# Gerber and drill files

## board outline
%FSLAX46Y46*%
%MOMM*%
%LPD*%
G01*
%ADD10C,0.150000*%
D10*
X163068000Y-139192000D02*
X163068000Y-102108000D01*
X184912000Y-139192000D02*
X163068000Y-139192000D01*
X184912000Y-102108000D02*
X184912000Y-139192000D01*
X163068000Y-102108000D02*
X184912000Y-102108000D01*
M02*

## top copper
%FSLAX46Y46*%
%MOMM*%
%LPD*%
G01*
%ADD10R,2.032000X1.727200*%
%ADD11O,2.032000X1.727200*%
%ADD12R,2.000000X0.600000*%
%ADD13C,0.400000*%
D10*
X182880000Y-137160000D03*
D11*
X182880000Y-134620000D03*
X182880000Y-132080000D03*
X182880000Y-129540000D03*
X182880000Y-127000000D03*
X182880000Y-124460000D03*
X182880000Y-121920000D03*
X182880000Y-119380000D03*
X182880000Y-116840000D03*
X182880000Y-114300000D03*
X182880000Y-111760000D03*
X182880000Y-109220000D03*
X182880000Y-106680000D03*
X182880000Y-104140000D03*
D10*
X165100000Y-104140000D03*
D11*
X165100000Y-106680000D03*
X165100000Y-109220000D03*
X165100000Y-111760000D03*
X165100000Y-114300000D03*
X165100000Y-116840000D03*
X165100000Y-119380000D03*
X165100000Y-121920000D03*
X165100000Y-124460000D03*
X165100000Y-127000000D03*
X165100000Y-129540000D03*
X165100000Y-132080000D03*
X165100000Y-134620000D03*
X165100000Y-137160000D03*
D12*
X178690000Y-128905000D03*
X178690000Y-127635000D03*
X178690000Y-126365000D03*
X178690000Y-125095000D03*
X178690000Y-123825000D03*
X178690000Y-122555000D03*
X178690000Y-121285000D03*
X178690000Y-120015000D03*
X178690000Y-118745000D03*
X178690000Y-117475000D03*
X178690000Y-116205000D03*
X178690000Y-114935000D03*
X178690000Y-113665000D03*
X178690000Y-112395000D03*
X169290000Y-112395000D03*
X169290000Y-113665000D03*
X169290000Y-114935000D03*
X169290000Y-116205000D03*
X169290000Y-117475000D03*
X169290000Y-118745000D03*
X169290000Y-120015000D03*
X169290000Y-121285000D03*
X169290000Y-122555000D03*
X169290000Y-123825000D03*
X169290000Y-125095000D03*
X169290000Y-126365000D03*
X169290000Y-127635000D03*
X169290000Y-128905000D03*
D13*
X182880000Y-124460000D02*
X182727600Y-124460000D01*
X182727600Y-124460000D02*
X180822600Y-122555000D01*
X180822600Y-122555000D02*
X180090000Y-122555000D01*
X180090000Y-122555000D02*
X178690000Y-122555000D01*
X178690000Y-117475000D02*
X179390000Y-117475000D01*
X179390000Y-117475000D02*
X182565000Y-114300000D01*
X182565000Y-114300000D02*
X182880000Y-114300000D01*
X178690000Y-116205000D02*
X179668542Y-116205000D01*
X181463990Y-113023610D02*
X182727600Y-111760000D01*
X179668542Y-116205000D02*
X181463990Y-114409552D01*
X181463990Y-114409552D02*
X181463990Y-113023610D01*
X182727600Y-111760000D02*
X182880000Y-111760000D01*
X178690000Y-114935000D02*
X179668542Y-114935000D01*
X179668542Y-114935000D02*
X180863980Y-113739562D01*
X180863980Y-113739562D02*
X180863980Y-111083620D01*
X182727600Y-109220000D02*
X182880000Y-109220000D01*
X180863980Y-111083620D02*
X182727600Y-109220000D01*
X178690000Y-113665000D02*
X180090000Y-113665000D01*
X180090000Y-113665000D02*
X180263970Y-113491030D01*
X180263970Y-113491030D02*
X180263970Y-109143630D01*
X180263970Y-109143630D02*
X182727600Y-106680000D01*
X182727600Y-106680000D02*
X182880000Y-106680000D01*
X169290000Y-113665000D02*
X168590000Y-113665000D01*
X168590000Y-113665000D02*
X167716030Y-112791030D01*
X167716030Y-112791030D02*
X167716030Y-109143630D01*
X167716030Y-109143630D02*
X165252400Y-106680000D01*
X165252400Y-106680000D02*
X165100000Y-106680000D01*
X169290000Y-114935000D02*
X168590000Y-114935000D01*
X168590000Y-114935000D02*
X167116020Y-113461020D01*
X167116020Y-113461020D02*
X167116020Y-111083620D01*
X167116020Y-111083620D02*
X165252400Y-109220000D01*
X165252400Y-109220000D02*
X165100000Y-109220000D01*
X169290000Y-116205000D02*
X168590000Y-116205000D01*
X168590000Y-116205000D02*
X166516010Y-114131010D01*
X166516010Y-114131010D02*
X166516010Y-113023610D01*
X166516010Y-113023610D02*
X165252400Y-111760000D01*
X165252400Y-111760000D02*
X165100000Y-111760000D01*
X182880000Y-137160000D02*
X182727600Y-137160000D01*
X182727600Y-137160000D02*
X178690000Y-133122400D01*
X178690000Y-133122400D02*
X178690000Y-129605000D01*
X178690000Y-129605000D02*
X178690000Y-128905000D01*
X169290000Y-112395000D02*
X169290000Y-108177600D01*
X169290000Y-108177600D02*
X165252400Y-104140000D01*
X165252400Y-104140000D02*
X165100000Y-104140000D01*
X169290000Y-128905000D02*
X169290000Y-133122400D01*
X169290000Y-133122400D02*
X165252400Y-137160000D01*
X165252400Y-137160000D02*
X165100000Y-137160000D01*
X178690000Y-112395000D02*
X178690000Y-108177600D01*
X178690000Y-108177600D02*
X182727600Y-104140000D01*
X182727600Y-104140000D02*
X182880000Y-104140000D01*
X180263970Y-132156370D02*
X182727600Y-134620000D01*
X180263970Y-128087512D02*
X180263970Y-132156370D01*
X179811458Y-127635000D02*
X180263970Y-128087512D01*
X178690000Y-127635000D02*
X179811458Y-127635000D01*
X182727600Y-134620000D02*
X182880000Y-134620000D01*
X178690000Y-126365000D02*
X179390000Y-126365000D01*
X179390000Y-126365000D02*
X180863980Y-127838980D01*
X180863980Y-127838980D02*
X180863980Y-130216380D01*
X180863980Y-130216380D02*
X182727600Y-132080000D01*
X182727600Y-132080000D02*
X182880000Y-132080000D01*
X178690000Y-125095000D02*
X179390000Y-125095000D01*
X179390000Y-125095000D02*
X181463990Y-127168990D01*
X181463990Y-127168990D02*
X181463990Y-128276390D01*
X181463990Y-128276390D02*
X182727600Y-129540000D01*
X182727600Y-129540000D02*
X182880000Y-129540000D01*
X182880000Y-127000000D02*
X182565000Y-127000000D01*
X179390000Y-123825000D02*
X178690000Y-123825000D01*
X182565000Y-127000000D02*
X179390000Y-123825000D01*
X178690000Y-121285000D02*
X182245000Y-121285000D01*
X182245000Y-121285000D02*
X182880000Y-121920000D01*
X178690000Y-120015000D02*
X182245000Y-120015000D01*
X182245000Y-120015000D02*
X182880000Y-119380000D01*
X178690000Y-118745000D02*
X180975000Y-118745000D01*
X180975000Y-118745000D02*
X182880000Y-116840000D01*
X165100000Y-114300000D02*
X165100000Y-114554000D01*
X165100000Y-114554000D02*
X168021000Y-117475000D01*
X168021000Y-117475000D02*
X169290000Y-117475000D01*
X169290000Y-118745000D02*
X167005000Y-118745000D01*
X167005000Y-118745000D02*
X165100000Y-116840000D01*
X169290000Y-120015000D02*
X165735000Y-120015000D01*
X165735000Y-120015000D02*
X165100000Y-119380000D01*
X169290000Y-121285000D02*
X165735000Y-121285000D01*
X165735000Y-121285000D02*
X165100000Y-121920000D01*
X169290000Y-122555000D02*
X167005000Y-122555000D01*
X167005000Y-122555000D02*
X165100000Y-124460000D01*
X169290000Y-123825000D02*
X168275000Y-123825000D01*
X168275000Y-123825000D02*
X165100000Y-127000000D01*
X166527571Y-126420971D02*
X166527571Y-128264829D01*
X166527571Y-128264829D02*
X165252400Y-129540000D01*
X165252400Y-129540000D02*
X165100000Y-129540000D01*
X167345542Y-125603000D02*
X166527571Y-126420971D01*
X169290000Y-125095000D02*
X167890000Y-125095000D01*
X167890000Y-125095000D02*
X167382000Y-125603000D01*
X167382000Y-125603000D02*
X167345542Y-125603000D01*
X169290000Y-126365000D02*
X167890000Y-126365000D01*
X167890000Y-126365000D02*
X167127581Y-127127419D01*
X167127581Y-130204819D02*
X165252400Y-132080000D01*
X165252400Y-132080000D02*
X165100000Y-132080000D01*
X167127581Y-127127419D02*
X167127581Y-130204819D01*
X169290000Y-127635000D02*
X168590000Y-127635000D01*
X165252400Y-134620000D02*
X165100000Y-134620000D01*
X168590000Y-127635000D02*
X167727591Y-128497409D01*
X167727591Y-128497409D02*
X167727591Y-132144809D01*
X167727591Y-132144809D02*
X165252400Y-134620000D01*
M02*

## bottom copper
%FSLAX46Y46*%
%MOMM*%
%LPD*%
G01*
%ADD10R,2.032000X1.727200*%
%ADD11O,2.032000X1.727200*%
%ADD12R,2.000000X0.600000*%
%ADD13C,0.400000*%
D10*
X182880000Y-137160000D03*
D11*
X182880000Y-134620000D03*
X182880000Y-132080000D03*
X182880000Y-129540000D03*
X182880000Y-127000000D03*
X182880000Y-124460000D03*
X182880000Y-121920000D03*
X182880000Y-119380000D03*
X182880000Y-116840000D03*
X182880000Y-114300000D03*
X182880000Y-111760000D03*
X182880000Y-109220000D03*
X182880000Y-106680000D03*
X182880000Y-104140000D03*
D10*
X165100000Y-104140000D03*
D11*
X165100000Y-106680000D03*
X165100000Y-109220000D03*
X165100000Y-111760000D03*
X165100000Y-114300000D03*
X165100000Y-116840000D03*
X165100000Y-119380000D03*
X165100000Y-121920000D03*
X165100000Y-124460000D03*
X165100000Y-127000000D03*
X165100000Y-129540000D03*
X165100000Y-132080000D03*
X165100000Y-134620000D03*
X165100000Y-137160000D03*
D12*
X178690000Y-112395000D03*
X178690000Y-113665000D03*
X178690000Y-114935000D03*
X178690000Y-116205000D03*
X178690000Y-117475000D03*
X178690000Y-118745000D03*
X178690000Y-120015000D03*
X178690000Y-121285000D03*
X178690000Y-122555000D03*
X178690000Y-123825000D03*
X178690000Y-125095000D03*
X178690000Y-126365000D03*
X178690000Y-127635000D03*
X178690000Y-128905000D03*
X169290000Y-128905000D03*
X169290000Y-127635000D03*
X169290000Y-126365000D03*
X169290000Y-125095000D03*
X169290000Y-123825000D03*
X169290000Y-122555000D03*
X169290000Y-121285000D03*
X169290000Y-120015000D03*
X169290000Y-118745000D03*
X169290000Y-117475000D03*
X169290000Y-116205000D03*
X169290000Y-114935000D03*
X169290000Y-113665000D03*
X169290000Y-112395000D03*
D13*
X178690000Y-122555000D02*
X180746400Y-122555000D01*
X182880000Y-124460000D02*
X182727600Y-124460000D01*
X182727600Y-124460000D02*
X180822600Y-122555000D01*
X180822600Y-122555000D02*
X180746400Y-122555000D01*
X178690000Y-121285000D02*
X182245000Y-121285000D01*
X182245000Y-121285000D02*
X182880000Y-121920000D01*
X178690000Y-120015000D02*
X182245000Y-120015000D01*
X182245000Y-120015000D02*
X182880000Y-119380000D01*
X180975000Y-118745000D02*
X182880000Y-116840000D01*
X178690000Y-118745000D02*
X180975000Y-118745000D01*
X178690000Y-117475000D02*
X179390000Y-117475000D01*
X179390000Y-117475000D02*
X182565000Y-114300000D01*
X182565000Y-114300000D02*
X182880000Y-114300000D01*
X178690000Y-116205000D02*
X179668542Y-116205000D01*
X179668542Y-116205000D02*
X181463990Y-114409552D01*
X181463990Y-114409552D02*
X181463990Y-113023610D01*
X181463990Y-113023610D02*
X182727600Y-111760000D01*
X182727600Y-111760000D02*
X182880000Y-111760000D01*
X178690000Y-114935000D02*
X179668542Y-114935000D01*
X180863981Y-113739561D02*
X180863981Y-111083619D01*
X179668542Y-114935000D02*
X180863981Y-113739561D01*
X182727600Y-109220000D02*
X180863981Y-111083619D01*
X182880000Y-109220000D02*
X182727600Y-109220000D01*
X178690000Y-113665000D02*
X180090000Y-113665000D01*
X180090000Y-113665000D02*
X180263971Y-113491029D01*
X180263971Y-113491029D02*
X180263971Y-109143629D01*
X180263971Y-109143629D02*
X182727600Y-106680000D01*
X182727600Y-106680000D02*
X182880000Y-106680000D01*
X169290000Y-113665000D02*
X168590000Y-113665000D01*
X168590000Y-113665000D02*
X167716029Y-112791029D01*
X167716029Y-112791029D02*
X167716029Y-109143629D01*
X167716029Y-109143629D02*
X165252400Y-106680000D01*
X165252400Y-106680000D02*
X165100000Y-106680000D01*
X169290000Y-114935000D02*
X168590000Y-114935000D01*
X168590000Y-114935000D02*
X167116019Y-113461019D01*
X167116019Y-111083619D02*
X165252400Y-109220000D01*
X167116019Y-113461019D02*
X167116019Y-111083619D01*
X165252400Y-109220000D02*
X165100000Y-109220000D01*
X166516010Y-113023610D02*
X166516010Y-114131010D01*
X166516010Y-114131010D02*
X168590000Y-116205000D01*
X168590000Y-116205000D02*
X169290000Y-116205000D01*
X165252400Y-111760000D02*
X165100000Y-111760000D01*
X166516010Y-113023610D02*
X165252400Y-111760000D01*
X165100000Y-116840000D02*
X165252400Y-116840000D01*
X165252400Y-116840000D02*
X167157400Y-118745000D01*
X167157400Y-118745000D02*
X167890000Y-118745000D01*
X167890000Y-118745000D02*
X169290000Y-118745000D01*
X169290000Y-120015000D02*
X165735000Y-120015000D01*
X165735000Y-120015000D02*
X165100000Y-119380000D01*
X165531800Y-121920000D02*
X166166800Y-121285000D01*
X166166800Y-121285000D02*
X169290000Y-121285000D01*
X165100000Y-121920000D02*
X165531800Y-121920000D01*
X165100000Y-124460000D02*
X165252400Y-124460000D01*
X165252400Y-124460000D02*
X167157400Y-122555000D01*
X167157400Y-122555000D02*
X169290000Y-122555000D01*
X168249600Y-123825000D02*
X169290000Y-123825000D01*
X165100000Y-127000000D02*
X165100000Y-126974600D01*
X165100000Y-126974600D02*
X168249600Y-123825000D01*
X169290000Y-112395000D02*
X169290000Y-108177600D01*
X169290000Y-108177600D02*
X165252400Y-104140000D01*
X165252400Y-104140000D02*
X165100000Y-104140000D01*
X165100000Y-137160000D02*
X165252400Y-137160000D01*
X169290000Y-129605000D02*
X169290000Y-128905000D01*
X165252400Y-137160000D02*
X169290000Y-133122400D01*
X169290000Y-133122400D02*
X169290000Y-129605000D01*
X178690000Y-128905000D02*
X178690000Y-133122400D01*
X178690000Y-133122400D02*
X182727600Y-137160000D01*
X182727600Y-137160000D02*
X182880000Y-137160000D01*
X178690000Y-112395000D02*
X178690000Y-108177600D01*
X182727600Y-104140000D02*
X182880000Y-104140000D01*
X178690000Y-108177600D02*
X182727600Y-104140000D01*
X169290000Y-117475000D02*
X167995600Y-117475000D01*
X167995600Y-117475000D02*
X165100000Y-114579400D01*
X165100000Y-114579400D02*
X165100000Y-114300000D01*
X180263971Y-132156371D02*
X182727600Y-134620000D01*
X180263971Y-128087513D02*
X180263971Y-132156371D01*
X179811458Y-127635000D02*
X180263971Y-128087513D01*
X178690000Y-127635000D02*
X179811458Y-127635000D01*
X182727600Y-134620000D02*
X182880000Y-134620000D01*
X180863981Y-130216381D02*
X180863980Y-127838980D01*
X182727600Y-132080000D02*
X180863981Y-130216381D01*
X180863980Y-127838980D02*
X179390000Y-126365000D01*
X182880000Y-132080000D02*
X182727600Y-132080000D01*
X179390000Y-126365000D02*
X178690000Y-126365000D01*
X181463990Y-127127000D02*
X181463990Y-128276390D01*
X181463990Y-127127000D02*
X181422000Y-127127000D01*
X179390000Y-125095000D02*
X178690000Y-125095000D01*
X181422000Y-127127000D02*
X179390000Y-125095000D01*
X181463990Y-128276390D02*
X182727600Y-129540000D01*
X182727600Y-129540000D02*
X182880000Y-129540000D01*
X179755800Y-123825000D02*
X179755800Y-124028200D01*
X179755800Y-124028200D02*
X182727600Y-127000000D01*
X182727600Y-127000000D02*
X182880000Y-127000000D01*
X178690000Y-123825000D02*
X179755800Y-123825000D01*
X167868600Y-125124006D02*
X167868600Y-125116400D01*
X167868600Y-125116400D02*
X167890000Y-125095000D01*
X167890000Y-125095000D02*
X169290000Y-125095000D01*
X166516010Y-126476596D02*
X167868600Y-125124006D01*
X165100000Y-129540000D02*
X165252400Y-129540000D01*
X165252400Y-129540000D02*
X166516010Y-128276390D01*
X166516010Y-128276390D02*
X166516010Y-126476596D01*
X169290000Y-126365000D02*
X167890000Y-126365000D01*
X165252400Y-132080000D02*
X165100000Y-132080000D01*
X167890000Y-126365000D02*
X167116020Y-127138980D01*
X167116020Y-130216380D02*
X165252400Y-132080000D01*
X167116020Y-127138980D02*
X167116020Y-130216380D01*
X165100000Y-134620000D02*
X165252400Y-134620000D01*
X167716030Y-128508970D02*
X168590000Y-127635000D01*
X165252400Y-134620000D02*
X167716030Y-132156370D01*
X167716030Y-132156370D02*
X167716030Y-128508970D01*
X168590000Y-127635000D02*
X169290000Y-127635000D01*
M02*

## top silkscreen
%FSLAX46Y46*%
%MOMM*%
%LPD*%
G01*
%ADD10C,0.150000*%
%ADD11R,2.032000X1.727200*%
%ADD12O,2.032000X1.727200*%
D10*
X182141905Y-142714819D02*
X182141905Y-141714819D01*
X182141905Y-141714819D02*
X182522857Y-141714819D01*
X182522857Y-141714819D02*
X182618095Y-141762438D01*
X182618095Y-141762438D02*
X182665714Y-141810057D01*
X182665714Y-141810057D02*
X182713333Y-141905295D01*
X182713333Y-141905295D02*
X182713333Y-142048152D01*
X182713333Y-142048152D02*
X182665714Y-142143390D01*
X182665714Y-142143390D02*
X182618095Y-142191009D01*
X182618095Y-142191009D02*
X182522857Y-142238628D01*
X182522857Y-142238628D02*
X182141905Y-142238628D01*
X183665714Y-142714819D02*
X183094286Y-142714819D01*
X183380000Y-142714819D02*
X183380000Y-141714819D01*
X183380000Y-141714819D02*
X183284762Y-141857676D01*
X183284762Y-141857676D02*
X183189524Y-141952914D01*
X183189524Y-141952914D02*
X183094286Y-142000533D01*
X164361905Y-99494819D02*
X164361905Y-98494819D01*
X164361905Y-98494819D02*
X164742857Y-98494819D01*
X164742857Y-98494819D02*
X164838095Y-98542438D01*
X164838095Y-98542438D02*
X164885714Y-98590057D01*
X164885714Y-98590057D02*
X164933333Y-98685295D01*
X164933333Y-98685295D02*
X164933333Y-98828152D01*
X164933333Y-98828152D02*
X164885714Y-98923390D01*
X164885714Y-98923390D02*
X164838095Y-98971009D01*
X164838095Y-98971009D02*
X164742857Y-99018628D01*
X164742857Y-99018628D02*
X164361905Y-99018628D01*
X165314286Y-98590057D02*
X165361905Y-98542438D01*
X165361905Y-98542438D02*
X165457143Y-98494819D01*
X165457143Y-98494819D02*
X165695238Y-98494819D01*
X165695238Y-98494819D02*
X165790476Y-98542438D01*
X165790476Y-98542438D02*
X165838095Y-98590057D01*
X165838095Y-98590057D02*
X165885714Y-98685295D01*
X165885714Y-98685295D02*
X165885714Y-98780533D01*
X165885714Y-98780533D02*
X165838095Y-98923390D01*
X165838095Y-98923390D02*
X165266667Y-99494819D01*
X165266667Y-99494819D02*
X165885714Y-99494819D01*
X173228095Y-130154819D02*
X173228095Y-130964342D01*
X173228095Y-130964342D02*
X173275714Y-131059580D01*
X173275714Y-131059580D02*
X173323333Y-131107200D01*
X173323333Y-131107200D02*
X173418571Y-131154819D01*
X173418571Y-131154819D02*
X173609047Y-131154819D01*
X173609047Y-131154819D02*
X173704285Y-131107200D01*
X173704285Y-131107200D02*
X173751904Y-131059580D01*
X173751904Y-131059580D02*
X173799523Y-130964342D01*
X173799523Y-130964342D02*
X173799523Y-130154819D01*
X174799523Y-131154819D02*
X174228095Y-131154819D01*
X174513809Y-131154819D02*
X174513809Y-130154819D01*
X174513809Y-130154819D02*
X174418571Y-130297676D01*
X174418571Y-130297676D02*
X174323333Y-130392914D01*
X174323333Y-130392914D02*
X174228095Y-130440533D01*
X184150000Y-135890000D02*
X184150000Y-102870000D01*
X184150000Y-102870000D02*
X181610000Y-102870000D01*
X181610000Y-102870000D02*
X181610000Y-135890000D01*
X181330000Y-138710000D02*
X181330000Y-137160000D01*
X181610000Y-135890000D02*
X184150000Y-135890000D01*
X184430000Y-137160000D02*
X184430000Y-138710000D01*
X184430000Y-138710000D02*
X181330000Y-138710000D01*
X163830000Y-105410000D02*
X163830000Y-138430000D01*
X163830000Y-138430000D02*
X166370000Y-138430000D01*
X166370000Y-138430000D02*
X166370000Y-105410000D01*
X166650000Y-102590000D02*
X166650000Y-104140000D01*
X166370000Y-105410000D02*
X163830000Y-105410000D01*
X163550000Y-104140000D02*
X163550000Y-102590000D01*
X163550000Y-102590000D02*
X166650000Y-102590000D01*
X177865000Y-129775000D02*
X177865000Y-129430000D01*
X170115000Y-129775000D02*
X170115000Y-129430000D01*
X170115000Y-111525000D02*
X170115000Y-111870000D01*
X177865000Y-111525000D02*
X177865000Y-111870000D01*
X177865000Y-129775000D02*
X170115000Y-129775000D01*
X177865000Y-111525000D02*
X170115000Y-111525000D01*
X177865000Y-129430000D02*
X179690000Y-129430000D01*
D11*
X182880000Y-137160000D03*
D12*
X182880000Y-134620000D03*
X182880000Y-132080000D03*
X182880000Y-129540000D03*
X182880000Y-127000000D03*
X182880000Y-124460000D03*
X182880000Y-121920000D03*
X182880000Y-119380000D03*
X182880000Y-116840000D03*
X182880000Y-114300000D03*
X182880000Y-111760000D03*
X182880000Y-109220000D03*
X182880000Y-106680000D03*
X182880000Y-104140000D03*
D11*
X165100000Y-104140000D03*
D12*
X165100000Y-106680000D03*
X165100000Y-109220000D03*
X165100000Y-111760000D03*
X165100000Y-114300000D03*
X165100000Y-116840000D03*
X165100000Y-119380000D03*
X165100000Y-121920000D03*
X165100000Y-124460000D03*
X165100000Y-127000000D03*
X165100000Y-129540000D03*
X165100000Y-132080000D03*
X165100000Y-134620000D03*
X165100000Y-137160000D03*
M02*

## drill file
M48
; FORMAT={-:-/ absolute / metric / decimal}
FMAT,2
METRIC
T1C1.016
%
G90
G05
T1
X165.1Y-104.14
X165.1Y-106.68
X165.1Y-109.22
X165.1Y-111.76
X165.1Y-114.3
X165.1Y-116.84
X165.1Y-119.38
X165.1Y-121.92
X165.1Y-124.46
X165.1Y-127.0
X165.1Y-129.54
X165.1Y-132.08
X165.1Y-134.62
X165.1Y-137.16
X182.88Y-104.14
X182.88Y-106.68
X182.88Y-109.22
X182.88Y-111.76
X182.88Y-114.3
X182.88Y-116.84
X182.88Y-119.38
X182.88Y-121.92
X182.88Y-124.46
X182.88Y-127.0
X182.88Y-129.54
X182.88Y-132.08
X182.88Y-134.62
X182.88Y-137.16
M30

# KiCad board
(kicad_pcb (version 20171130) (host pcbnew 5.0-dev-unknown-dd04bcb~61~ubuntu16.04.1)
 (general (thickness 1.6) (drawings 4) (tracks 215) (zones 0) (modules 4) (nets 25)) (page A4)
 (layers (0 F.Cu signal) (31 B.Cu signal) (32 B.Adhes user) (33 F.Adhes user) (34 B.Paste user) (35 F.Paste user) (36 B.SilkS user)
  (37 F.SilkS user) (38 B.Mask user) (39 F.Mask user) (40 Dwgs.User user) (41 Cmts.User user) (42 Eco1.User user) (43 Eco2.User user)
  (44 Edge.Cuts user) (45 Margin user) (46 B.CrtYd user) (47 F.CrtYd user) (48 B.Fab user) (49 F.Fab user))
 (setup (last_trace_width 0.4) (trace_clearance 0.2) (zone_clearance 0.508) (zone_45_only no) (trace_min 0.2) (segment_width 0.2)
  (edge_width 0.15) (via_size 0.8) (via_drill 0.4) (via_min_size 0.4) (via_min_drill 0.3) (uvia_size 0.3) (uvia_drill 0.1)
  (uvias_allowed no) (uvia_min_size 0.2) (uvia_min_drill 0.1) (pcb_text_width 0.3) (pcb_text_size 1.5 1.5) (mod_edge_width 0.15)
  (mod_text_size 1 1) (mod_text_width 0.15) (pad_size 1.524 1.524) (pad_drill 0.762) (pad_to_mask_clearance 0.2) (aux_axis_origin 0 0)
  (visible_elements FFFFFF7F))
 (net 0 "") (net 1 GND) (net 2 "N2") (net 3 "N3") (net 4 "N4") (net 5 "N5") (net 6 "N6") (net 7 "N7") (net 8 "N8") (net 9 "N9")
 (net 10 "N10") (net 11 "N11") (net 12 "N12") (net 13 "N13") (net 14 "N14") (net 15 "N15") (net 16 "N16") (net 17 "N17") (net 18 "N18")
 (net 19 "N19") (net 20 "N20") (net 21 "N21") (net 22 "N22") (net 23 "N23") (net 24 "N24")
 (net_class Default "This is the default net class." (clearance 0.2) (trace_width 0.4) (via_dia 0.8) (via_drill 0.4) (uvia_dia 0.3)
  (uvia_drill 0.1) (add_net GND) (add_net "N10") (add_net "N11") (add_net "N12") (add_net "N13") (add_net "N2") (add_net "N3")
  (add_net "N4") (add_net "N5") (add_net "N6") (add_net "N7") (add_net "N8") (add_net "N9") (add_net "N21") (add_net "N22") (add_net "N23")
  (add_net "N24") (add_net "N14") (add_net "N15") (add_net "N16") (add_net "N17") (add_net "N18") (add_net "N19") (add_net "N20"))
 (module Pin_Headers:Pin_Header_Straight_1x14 (layer F.Cu) (at 182.88 137.16 180)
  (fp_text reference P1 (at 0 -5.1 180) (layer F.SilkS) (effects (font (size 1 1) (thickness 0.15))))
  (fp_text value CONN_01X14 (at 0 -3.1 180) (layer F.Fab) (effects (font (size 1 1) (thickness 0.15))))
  (fp_line (start -1.27 1.27) (end -1.27 34.29) (layer F.SilkS) (width 0.15))
  (fp_line (start -1.27 34.29) (end 1.27 34.29) (layer F.SilkS) (width 0.15))
  (fp_line (start 1.27 34.29) (end 1.27 1.27) (layer F.SilkS) (width 0.15))
  (fp_line (start 1.55 -1.55) (end 1.55 0) (layer F.SilkS) (width 0.15))
  (fp_line (start 1.27 1.27) (end -1.27 1.27) (layer F.SilkS) (width 0.15))
  (fp_line (start -1.55 0) (end -1.55 -1.55) (layer F.SilkS) (width 0.15))
  (fp_line (start -1.55 -1.55) (end 1.55 -1.55) (layer F.SilkS) (width 0.15))
  (pad 1 thru_hole rect (at 0 0 180) (size 2.032 1.7272) (drill 1.016) (layers *.Cu *.Mask F.SilkS) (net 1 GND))
  (pad 2 thru_hole oval (at 0 2.54 180) (size 2.032 1.7272) (drill 1.016) (layers *.Cu *.Mask F.SilkS) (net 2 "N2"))
  (pad 3 thru_hole oval (at 0 5.08 180) (size 2.032 1.7272) (drill 1.016) (layers *.Cu *.Mask F.SilkS) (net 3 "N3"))
  (pad 4 thru_hole oval (at 0 7.62 180) (size 2.032 1.7272) (drill 1.016) (layers *.Cu *.Mask F.SilkS) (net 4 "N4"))
  (pad 5 thru_hole oval (at 0 10.16 180) (size 2.032 1.7272) (drill 1.016) (layers *.Cu *.Mask F.SilkS) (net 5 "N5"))
  (pad 6 thru_hole oval (at 0 12.7 180) (size 2.032 1.7272) (drill 1.016) (layers *.Cu *.Mask F.SilkS) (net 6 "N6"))
  (pad 7 thru_hole oval (at 0 15.24 180) (size 2.032 1.7272) (drill 1.016) (layers *.Cu *.Mask F.SilkS) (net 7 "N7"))
  (pad 8 thru_hole oval (at 0 17.78 180) (size 2.032 1.7272) (drill 1.016) (layers *.Cu *.Mask F.SilkS) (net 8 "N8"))
  (pad 9 thru_hole oval (at 0 20.32 180) (size 2.032 1.7272) (drill 1.016) (layers *.Cu *.Mask F.SilkS) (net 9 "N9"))
  (pad 10 thru_hole oval (at 0 22.86 180) (size 2.032 1.7272) (drill 1.016) (layers *.Cu *.Mask F.SilkS) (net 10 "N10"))
  (pad 11 thru_hole oval (at 0 25.4 180) (size 2.032 1.7272) (drill 1.016) (layers *.Cu *.Mask F.SilkS) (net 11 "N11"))
  (pad 12 thru_hole oval (at 0 27.94 180) (size 2.032 1.7272) (drill 1.016) (layers *.Cu *.Mask F.SilkS) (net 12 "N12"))
  (pad 13 thru_hole oval (at 0 30.48 180) (size 2.032 1.7272) (drill 1.016) (layers *.Cu *.Mask F.SilkS) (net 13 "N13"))
  (pad 14 thru_hole oval (at 0 33.02 180) (size 2.032 1.7272) (drill 1.016) (layers *.Cu *.Mask F.SilkS) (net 1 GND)))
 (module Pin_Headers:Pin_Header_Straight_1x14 (layer F.Cu) (at 165.1 104.14)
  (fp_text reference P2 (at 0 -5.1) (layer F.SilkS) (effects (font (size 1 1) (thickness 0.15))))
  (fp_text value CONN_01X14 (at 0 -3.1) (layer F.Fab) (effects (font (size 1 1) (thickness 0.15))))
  (fp_line (start -1.27 1.27) (end -1.27 34.29) (layer F.SilkS) (width 0.15))
  (fp_line (start -1.27 34.29) (end 1.27 34.29) (layer F.SilkS) (width 0.15))
  (fp_line (start 1.27 34.29) (end 1.27 1.27) (layer F.SilkS) (width 0.15))
  (fp_line (start 1.55 -1.55) (end 1.55 0) (layer F.SilkS) (width 0.15))
  (fp_line (start 1.27 1.27) (end -1.27 1.27) (layer F.SilkS) (width 0.15))
  (fp_line (start -1.55 0) (end -1.55 -1.55) (layer F.SilkS) (width 0.15))
  (fp_line (start -1.55 -1.55) (end 1.55 -1.55) (layer F.SilkS) (width 0.15))
  (pad 1 thru_hole rect (at 0 0) (size 2.032 1.7272) (drill 1.016) (layers *.Cu *.Mask F.SilkS) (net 1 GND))
  (pad 2 thru_hole oval (at 0 2.54) (size 2.032 1.7272) (drill 1.016) (layers *.Cu *.Mask F.SilkS) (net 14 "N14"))
  (pad 3 thru_hole oval (at 0 5.08) (size 2.032 1.7272) (drill 1.016) (layers *.Cu *.Mask F.SilkS) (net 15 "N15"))
  (pad 4 thru_hole oval (at 0 7.62) (size 2.032 1.7272) (drill 1.016) (layers *.Cu *.Mask F.SilkS) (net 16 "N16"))
  (pad 5 thru_hole oval (at 0 10.16) (size 2.032 1.7272) (drill 1.016) (layers *.Cu *.Mask F.SilkS) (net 2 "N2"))
  (pad 6 thru_hole oval (at 0 12.7) (size 2.032 1.7272) (drill 1.016) (layers *.Cu *.Mask F.SilkS) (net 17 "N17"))
  (pad 7 thru_hole oval (at 0 15.24) (size 2.032 1.7272) (drill 1.016) (layers *.Cu *.Mask F.SilkS) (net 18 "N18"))
  (pad 8 thru_hole oval (at 0 17.78) (size 2.032 1.7272) (drill 1.016) (layers *.Cu *.Mask F.SilkS) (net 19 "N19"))
  (pad 9 thru_hole oval (at 0 20.32) (size 2.032 1.7272) (drill 1.016) (layers *.Cu *.Mask F.SilkS) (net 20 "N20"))
  (pad 10 thru_hole oval (at 0 22.86) (size 2.032 1.7272) (drill 1.016) (layers *.Cu *.Mask F.SilkS) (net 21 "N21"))
  (pad 11 thru_hole oval (at 0 25.4) (size 2.032 1.7272) (drill 1.016) (layers *.Cu *.Mask F.SilkS) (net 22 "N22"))
  (pad 12 thru_hole oval (at 0 27.94) (size 2.032 1.7272) (drill 1.016) (layers *.Cu *.Mask F.SilkS) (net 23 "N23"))
  (pad 13 thru_hole oval (at 0 30.48) (size 2.032 1.7272) (drill 1.016) (layers *.Cu *.Mask F.SilkS) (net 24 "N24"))
  (pad 14 thru_hole oval (at 0 33.02) (size 2.032 1.7272) (drill 1.016) (layers *.Cu *.Mask F.SilkS) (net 1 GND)))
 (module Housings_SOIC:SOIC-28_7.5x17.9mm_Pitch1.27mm (layer F.Cu) (at 173.99 120.65 180)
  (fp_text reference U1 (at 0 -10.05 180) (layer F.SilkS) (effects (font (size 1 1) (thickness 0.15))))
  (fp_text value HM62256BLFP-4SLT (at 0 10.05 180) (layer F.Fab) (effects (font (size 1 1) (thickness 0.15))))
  (fp_line (start -3.875 -9.125) (end -3.875 -8.78) (layer F.SilkS) (width 0.15))
  (fp_line (start 3.875 -9.125) (end 3.875 -8.78) (layer F.SilkS) (width 0.15))
  (fp_line (start 3.875 9.125) (end 3.875 8.78) (layer F.SilkS) (width 0.15))
  (fp_line (start -3.875 9.125) (end -3.875 8.78) (layer F.SilkS) (width 0.15))
  (fp_line (start -3.875 -9.125) (end 3.875 -9.125) (layer F.SilkS) (width 0.15))
  (fp_line (start -3.875 9.125) (end 3.875 9.125) (layer F.SilkS) (width 0.15))
  (fp_line (start -3.875 -8.78) (end -5.7 -8.78) (layer F.SilkS) (width 0.15))
  (pad 1 smd rect (at -4.7 -8.255 180) (size 2 0.6) (layers F.Cu F.Paste F.Mask) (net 1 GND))
  (pad 2 smd rect (at -4.7 -6.985 180) (size 2 0.6) (layers F.Cu F.Paste F.Mask) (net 2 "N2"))
  (pad 3 smd rect (at -4.7 -5.715 180) (size 2 0.6) (layers F.Cu F.Paste F.Mask) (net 3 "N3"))
  (pad 4 smd rect (at -4.7 -4.445 180) (size 2 0.6) (layers F.Cu F.Paste F.Mask) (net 4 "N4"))
  (pad 5 smd rect (at -4.7 -3.175 180) (size 2 0.6) (layers F.Cu F.Paste F.Mask) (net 5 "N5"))
  (pad 6 smd rect (at -4.7 -1.905 180) (size 2 0.6) (layers F.Cu F.Paste F.Mask) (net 6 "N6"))
  (pad 7 smd rect (at -4.7 -0.635 180) (size 2 0.6) (layers F.Cu F.Paste F.Mask) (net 7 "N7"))
  (pad 8 smd rect (at -4.7 0.635 180) (size 2 0.6) (layers F.Cu F.Paste F.Mask) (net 8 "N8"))
  (pad 9 smd rect (at -4.7 1.905 180) (size 2 0.6) (layers F.Cu F.Paste F.Mask) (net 9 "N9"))
  (pad 10 smd rect (at -4.7 3.175 180) (size 2 0.6) (layers F.Cu F.Paste F.Mask) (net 10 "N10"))
  (pad 11 smd rect (at -4.7 4.445 180) (size 2 0.6) (layers F.Cu F.Paste F.Mask) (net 11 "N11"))
  (pad 12 smd rect (at -4.7 5.715 180) (size 2 0.6) (layers F.Cu F.Paste F.Mask) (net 12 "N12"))
  (pad 13 smd rect (at -4.7 6.985 180) (size 2 0.6) (layers F.Cu F.Paste F.Mask) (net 13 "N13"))
  (pad 14 smd rect (at -4.7 8.255 180) (size 2 0.6) (layers F.Cu F.Paste F.Mask) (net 1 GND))
  (pad 15 smd rect (at 4.7 8.255 180) (size 2 0.6) (layers F.Cu F.Paste F.Mask) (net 1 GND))
  (pad 16 smd rect (at 4.7 6.985 180) (size 2 0.6) (layers F.Cu F.Paste F.Mask) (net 14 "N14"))
  (pad 17 smd rect (at 4.7 5.715 180) (size 2 0.6) (layers F.Cu F.Paste F.Mask) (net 15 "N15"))
  (pad 18 smd rect (at 4.7 4.445 180) (size 2 0.6) (layers F.Cu F.Paste F.Mask) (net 16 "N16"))
  (pad 19 smd rect (at 4.7 3.175 180) (size 2 0.6) (layers F.Cu F.Paste F.Mask) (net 2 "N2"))
  (pad 20 smd rect (at 4.7 1.905 180) (size 2 0.6) (layers F.Cu F.Paste F.Mask) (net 17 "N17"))
  (pad 21 smd rect (at 4.7 0.635 180) (size 2 0.6) (layers F.Cu F.Paste F.Mask) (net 18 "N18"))
  (pad 22 smd rect (at 4.7 -0.635 180) (size 2 0.6) (layers F.Cu F.Paste F.Mask) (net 19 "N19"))
  (pad 23 smd rect (at 4.7 -1.905 180) (size 2 0.6) (layers F.Cu F.Paste F.Mask) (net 20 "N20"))
  (pad 24 smd rect (at 4.7 -3.175 180) (size 2 0.6) (layers F.Cu F.Paste F.Mask) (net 21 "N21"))
  (pad 25 smd rect (at 4.7 -4.445 180) (size 2 0.6) (layers F.Cu F.Paste F.Mask) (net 22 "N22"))
  (pad 26 smd rect (at 4.7 -5.715 180) (size 2 0.6) (layers F.Cu F.Paste F.Mask) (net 23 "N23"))
  (pad 27 smd rect (at 4.7 -6.985 180) (size 2 0.6) (layers F.Cu F.Paste F.Mask) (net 24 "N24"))
  (pad 28 smd rect (at 4.7 -8.255 180) (size 2 0.6) (layers F.Cu F.Paste F.Mask) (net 1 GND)))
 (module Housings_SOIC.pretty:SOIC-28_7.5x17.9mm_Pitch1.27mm (layer B.Cu) (at 173.99 120.65 180)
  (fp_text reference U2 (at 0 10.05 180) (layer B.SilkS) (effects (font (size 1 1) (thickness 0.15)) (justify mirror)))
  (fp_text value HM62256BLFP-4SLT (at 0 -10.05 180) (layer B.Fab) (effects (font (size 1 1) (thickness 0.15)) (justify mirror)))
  (pad 1 smd rect (at -4.7 8.255 180) (size 2 0.6) (layers B.Cu B.Paste B.Mask) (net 1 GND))
  (pad 2 smd rect (at -4.7 6.985 180) (size 2 0.6) (layers B.Cu B.Paste B.Mask) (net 13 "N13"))
  (pad 3 smd rect (at -4.7 5.715 180) (size 2 0.6) (layers B.Cu B.Paste B.Mask) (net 12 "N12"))
  (pad 4 smd rect (at -4.7 4.445 180) (size 2 0.6) (layers B.Cu B.Paste B.Mask) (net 11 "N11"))
  (pad 5 smd rect (at -4.7 3.175 180) (size 2 0.6) (layers B.Cu B.Paste B.Mask) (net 10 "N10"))
  (pad 6 smd rect (at -4.7 1.905 180) (size 2 0.6) (layers B.Cu B.Paste B.Mask) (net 9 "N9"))
  (pad 7 smd rect (at -4.7 0.635 180) (size 2 0.6) (layers B.Cu B.Paste B.Mask) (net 8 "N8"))
  (pad 8 smd rect (at -4.7 -0.635 180) (size 2 0.6) (layers B.Cu B.Paste B.Mask) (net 7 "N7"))
  (pad 9 smd rect (at -4.7 -1.905 180) (size 2 0.6) (layers B.Cu B.Paste B.Mask) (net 6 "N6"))
  (pad 10 smd rect (at -4.7 -3.175 180) (size 2 0.6) (layers B.Cu B.Paste B.Mask) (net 5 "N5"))
  (pad 11 smd rect (at -4.7 -4.445 180) (size 2 0.6) (layers B.Cu B.Paste B.Mask) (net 4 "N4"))
  (pad 12 smd rect (at -4.7 -5.715 180) (size 2 0.6) (layers B.Cu B.Paste B.Mask) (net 3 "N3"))
  (pad 13 smd rect (at -4.7 -6.985 180) (size 2 0.6) (layers B.Cu B.Paste B.Mask) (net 2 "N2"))
  (pad 14 smd rect (at -4.7 -8.255 180) (size 2 0.6) (layers B.Cu B.Paste B.Mask) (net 1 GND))
  (pad 15 smd rect (at 4.7 -8.255 180) (size 2 0.6) (layers B.Cu B.Paste B.Mask) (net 1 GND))
  (pad 16 smd rect (at 4.7 -6.985 180) (size 2 0.6) (layers B.Cu B.Paste B.Mask) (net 24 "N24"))
  (pad 17 smd rect (at 4.7 -5.715 180) (size 2 0.6) (layers B.Cu B.Paste B.Mask) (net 23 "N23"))
  (pad 18 smd rect (at 4.7 -4.445 180) (size 2 0.6) (layers B.Cu B.Paste B.Mask) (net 22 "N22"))
  (pad 19 smd rect (at 4.7 -3.175 180) (size 2 0.6) (layers B.Cu B.Paste B.Mask) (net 21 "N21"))
  (pad 20 smd rect (at 4.7 -1.905 180) (size 2 0.6) (layers B.Cu B.Paste B.Mask) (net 20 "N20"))
  (pad 21 smd rect (at 4.7 -0.635 180) (size 2 0.6) (layers B.Cu B.Paste B.Mask) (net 19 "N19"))
  (pad 22 smd rect (at 4.7 0.635 180) (size 2 0.6) (layers B.Cu B.Paste B.Mask) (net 18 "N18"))
  (pad 23 smd rect (at 4.7 1.905 180) (size 2 0.6) (layers B.Cu B.Paste B.Mask) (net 17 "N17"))
  (pad 24 smd rect (at 4.7 3.175 180) (size 2 0.6) (layers B.Cu B.Paste B.Mask) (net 2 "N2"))
  (pad 25 smd rect (at 4.7 4.445 180) (size 2 0.6) (layers B.Cu B.Paste B.Mask) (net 16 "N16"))
  (pad 26 smd rect (at 4.7 5.715 180) (size 2 0.6) (layers B.Cu B.Paste B.Mask) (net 15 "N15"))
  (pad 27 smd rect (at 4.7 6.985 180) (size 2 0.6) (layers B.Cu B.Paste B.Mask) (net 14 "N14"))
  (pad 28 smd rect (at 4.7 8.255 180) (size 2 0.6) (layers B.Cu B.Paste B.Mask) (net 1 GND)))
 (gr_line (start 163.068 139.192) (end 163.068 102.108) (angle 90) (layer Edge.Cuts) (width 0.15))
 (gr_line (start 184.912 139.192) (end 163.068 139.192) (angle 90) (layer Edge.Cuts) (width 0.15))
 (gr_line (start 184.912 102.108) (end 184.912 139.192) (angle 90) (layer Edge.Cuts) (width 0.15))
 (gr_line (start 163.068 102.108) (end 184.912 102.108) (angle 90) (layer Edge.Cuts) (width 0.15))
 (segment (start 178.69 122.555) (end 180.7464 122.555) (width 0.4) (layer B.Cu) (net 6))
 (segment (start 182.88 124.46) (end 182.7276 124.46) (width 0.4) (layer B.Cu) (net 6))
 (segment (start 182.7276 124.46) (end 180.8226 122.555) (width 0.4) (layer B.Cu) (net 6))
 (segment (start 180.8226 122.555) (end 180.7464 122.555) (width 0.4) (layer B.Cu) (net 6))
 (segment (start 182.88 124.46) (end 182.7276 124.46) (width 0.4) (layer F.Cu) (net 6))
 (segment (start 182.7276 124.46) (end 180.8226 122.555) (width 0.4) (layer F.Cu) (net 6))
 (segment (start 180.8226 122.555) (end 180.09 122.555) (width 0.4) (layer F.Cu) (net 6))
 (segment (start 180.09 122.555) (end 178.69 122.555) (width 0.4) (layer F.Cu) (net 6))
 (segment (start 178.69 121.285) (end 182.245 121.285) (width 0.4) (layer B.Cu) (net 7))
 (segment (start 182.245 121.285) (end 182.88 121.92) (width 0.4) (layer B.Cu) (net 7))
 (segment (start 178.69 120.015) (end 182.245 120.015) (width 0.4) (layer B.Cu) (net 8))
 (segment (start 182.245 120.015) (end 182.88 119.38) (width 0.4) (layer B.Cu) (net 8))
 (segment (start 180.975 118.745) (end 182.88 116.84) (width 0.4) (layer B.Cu) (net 9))
 (segment (start 178.69 118.745) (end 180.975 118.745) (width 0.4) (layer B.Cu) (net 9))
 (segment (start 178.69 117.475) (end 179.39 117.475) (width 0.4) (layer B.Cu) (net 10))
 (segment (start 179.39 117.475) (end 182.565 114.3) (width 0.4) (layer B.Cu) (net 10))
 (segment (start 182.565 114.3) (end 182.88 114.3) (width 0.4) (layer B.Cu) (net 10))
 (segment (start 178.69 117.475) (end 179.39 117.475) (width 0.4) (layer F.Cu) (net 10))
 (segment (start 179.39 117.475) (end 182.565 114.3) (width 0.4) (layer F.Cu) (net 10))
 (segment (start 182.565 114.3) (end 182.88 114.3) (width 0.4) (layer F.Cu) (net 10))
 (segment (start 178.69 116.205) (end 179.668542 116.205) (width 0.4) (layer B.Cu) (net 11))
 (segment (start 179.668542 116.205) (end 181.46399 114.409552) (width 0.4) (layer B.Cu) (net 11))
 (segment (start 181.46399 114.409552) (end 181.46399 113.02361) (width 0.4) (layer B.Cu) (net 11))
 (segment (start 181.46399 113.02361) (end 182.7276 111.76) (width 0.4) (layer B.Cu) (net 11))
 (segment (start 182.7276 111.76) (end 182.88 111.76) (width 0.4) (layer B.Cu) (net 11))
 (segment (start 178.69 116.205) (end 179.668542 116.205) (width 0.4) (layer F.Cu) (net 11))
 (segment (start 181.46399 113.02361) (end 182.7276 111.76) (width 0.4) (layer F.Cu) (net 11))
 (segment (start 179.668542 116.205) (end 181.46399 114.409552) (width 0.4) (layer F.Cu) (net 11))
 (segment (start 181.46399 114.409552) (end 181.46399 113.02361) (width 0.4) (layer F.Cu) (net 11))
 (segment (start 182.7276 111.76) (end 182.88 111.76) (width 0.4) (layer F.Cu) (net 11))
 (segment (start 178.69 114.935) (end 179.668542 114.935) (width 0.4) (layer B.Cu) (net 12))
 (segment (start 180.863981 113.739561) (end 180.863981 111.083619) (width 0.4) (layer B.Cu) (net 12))
 (segment (start 179.668542 114.935) (end 180.863981 113.739561) (width 0.4) (layer B.Cu) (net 12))
 (segment (start 182.7276 109.22) (end 180.863981 111.083619) (width 0.4) (layer B.Cu) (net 12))
 (segment (start 182.88 109.22) (end 182.7276 109.22) (width 0.4) (layer B.Cu) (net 12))
 (segment (start 178.69 114.935) (end 179.668542 114.935) (width 0.4) (layer F.Cu) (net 12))
 (segment (start 179.668542 114.935) (end 180.86398 113.739562) (width 0.4) (layer F.Cu) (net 12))
 (segment (start 180.86398 113.739562) (end 180.86398 111.08362) (width 0.4) (layer F.Cu) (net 12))
 (segment (start 182.7276 109.22) (end 182.88 109.22) (width 0.4) (layer F.Cu) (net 12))
 (segment (start 180.86398 111.08362) (end 182.7276 109.22) (width 0.4) (layer F.Cu) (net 12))
 (segment (start 178.69 113.665) (end 180.09 113.665) (width 0.4) (layer B.Cu) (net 13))
 (segment (start 180.09 113.665) (end 180.263971 113.491029) (width 0.4) (layer B.Cu) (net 13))
 (segment (start 180.263971 113.491029) (end 180.263971 109.143629) (width 0.4) (layer B.Cu) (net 13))
 (segment (start 180.263971 109.143629) (end 182.7276 106.68) (width 0.4) (layer B.Cu) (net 13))
 (segment (start 182.7276 106.68) (end 182.88 106.68) (width 0.4) (layer B.Cu) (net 13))
 (segment (start 178.69 113.665) (end 180.09 113.665) (width 0.4) (layer F.Cu) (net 13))
 (segment (start 180.09 113.665) (end 180.26397 113.49103) (width 0.4) (layer F.Cu) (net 13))
 (segment (start 180.26397 113.49103) (end 180.26397 109.14363) (width 0.4) (layer F.Cu) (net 13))
 (segment (start 180.26397 109.14363) (end 182.7276 106.68) (width 0.4) (layer F.Cu) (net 13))
 (segment (start 182.7276 106.68) (end 182.88 106.68) (width 0.4) (layer F.Cu) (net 13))
 (segment (start 169.29 113.665) (end 168.59 113.665) (width 0.4) (layer B.Cu) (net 14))
 (segment (start 168.59 113.665) (end 167.716029 112.791029) (width 0.4) (layer B.Cu) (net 14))
 (segment (start 167.716029 112.791029) (end 167.716029 109.143629) (width 0.4) (layer B.Cu) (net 14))
 (segment (start 167.716029 109.143629) (end 165.2524 106.68) (width 0.4) (layer B.Cu) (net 14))
 (segment (start 165.2524 106.68) (end 165.1 106.68) (width 0.4) (layer B.Cu) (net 14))
 (segment (start 169.29 113.665) (end 168.59 113.665) (width 0.4) (layer F.Cu) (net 14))
 (segment (start 168.59 113.665) (end 167.71603 112.79103) (width 0.4) (layer F.Cu) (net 14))
 (segment (start 167.71603 112.79103) (end 167.71603 109.14363) (width 0.4) (layer F.Cu) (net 14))
 (segment (start 167.71603 109.14363) (end 165.2524 106.68) (width 0.4) (layer F.Cu) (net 14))
 (segment (start 165.2524 106.68) (end 165.1 106.68) (width 0.4) (layer F.Cu) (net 14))
 (segment (start 169.29 114.935) (end 168.59 114.935) (width 0.4) (layer B.Cu) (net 15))
 (segment (start 168.59 114.935) (end 167.116019 113.461019) (width 0.4) (layer B.Cu) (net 15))
 (segment (start 167.116019 111.083619) (end 165.2524 109.22) (width 0.4) (layer B.Cu) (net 15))
 (segment (start 167.116019 113.461019) (end 167.116019 111.083619) (width 0.4) (layer B.Cu) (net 15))
 (segment (start 165.2524 109.22) (end 165.1 109.22) (width 0.4) (layer B.Cu) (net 15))
 (segment (start 169.29 114.935) (end 168.59 114.935) (width 0.4) (layer F.Cu) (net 15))
 (segment (start 168.59 114.935) (end 167.11602 113.46102) (width 0.4) (layer F.Cu) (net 15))
 (segment (start 167.11602 113.46102) (end 167.11602 111.08362) (width 0.4) (layer F.Cu) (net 15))
 (segment (start 167.11602 111.08362) (end 165.2524 109.22) (width 0.4) (layer F.Cu) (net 15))
 (segment (start 165.2524 109.22) (end 165.1 109.22) (width 0.4) (layer F.Cu) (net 15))
 (segment (start 166.51601 113.02361) (end 166.51601 114.13101) (width 0.4) (layer B.Cu) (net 16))
 (segment (start 166.51601 114.13101) (end 168.59 116.205) (width 0.4) (layer B.Cu) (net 16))
 (segment (start 168.59 116.205) (end 169.29 116.205) (width 0.4) (layer B.Cu) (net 16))
 (segment (start 165.2524 111.76) (end 165.1 111.76) (width 0.4) (layer B.Cu) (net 16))
 (segment (start 166.51601 113.02361) (end 165.2524 111.76) (width 0.4) (layer B.Cu) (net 16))
 (segment (start 169.29 116.205) (end 168.59 116.205) (width 0.4) (layer F.Cu) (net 16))
 (segment (start 168.59 116.205) (end 166.51601 114.13101) (width 0.4) (layer F.Cu) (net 16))
 (segment (start 166.51601 114.13101) (end 166.51601 113.02361) (width 0.4) (layer F.Cu) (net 16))
 (segment (start 166.51601 113.02361) (end 165.2524 111.76) (width 0.4) (layer F.Cu) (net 16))
 (segment (start 165.2524 111.76) (end 165.1 111.76) (width 0.4) (layer F.Cu) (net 16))
 (segment (start 165.1 116.84) (end 165.2524 116.84) (width 0.4) (layer B.Cu) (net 17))
 (segment (start 165.2524 116.84) (end 167.1574 118.745) (width 0.4) (layer B.Cu) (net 17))
 (segment (start 167.1574 118.745) (end 167.89 118.745) (width 0.4) (layer B.Cu) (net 17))
 (segment (start 167.89 118.745) (end 169.29 118.745) (width 0.4) (layer B.Cu) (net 17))
 (segment (start 169.29 120.015) (end 165.735 120.015) (width 0.4) (layer B.Cu) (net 18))
 (segment (start 165.735 120.015) (end 165.1 119.38) (width 0.4) (layer B.Cu) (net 18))
 (segment (start 165.5318 121.92) (end 166.1668 121.285) (width 0.4) (layer B.Cu) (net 19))
 (segment (start 166.1668 121.285) (end 169.29 121.285) (width 0.4) (layer B.Cu) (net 19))
 (segment (start 165.1 121.92) (end 165.5318 121.92) (width 0.4) (layer B.Cu) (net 19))
 (segment (start 165.1 124.46) (end 165.2524 124.46) (width 0.4) (layer B.Cu) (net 20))
 (segment (start 165.2524 124.46) (end 167.1574 122.555) (width 0.4) (layer B.Cu) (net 20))
 (segment (start 167.1574 122.555) (end 169.29 122.555) (width 0.4) (layer B.Cu) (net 20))
 (segment (start 168.2496 123.825) (end 169.29 123.825) (width 0.4) (layer B.Cu) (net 21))
 (segment (start 165.1 127) (end 165.1 126.9746) (width 0.4) (layer B.Cu) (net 21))
 (segment (start 165.1 126.9746) (end 168.2496 123.825) (width 0.4) (layer B.Cu) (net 21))
 (segment (start 182.88 137.16) (end 182.7276 137.16) (width 0.4) (layer F.Cu) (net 1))
 (segment (start 182.7276 137.16) (end 178.69 133.1224) (width 0.4) (layer F.Cu) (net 1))
 (segment (start 178.69 133.1224) (end 178.69 129.605) (width 0.4) (layer F.Cu) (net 1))
 (segment (start 178.69 129.605) (end 178.69 128.905) (width 0.4) (layer F.Cu) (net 1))
 (segment (start 169.29 112.395) (end 169.29 108.1776) (width 0.4) (layer B.Cu) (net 1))
 (segment (start 169.29 108.1776) (end 165.2524 104.14) (width 0.4) (layer B.Cu) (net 1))
 (segment (start 165.2524 104.14) (end 165.1 104.14) (width 0.4) (layer B.Cu) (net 1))
 (segment (start 165.1 137.16) (end 165.2524 137.16) (width 0.4) (layer B.Cu) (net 1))
 (segment (start 169.29 129.605) (end 169.29 128.905) (width 0.4) (layer B.Cu) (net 1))
 (segment (start 165.2524 137.16) (end 169.29 133.1224) (width 0.4) (layer B.Cu) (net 1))
 (segment (start 169.29 133.1224) (end 169.29 129.605) (width 0.4) (layer B.Cu) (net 1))
 (segment (start 178.69 128.905) (end 178.69 133.1224) (width 0.4) (layer B.Cu) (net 1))
 (segment (start 178.69 133.1224) (end 182.7276 137.16) (width 0.4) (layer B.Cu) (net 1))
 (segment (start 182.7276 137.16) (end 182.88 137.16) (width 0.4) (layer B.Cu) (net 1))
 (segment (start 178.69 112.395) (end 178.69 108.1776) (width 0.4) (layer B.Cu) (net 1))
 (segment (start 182.7276 104.14) (end 182.88 104.14) (width 0.4) (layer B.Cu) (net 1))
 (segment (start 178.69 108.1776) (end 182.7276 104.14) (width 0.4) (layer B.Cu) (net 1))
 (segment (start 169.29 112.395) (end 169.29 108.1776) (width 0.4) (layer F.Cu) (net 1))
 (segment (start 169.29 108.1776) (end 165.2524 104.14) (width 0.4) (layer F.Cu) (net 1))
 (segment (start 165.2524 104.14) (end 165.1 104.14) (width 0.4) (layer F.Cu) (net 1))
 (segment (start 169.29 128.905) (end 169.29 133.1224) (width 0.4) (layer F.Cu) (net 1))
 (segment (start 169.29 133.1224) (end 165.2524 137.16) (width 0.4) (layer F.Cu) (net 1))
 (segment (start 165.2524 137.16) (end 165.1 137.16) (width 0.4) (layer F.Cu) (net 1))
 (segment (start 178.69 112.395) (end 178.69 108.1776) (width 0.4) (layer F.Cu) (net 1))
 (segment (start 178.69 108.1776) (end 182.7276 104.14) (width 0.4) (layer F.Cu) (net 1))
 (segment (start 182.7276 104.14) (end 182.88 104.14) (width 0.4) (layer F.Cu) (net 1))
 (segment (start 169.29 117.475) (end 167.9956 117.475) (width 0.4) (layer B.Cu) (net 2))
 (segment (start 167.9956 117.475) (end 165.1 114.5794) (width 0.4) (layer B.Cu) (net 2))
 (segment (start 165.1 114.5794) (end 165.1 114.3) (width 0.4) (layer B.Cu) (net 2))
 (segment (start 180.26397 132.15637) (end 182.7276 134.62) (width 0.4) (layer F.Cu) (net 2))
 (segment (start 180.26397 128.087512) (end 180.26397 132.15637) (width 0.4) (layer F.Cu) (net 2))
 (segment (start 179.811458 127.635) (end 180.26397 128.087512) (width 0.4) (layer F.Cu) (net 2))
 (segment (start 178.69 127.635) (end 179.811458 127.635) (width 0.4) (layer F.Cu) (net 2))
 (segment (start 182.7276 134.62) (end 182.88 134.62) (width 0.4) (layer F.Cu) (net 2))
 (segment (start 180.263971 132.156371) (end 182.7276 134.62) (width 0.4) (layer B.Cu) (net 2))
 (segment (start 180.263971 128.087513) (end 180.263971 132.156371) (width 0.4) (layer B.Cu) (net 2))
 (segment (start 179.811458 127.635) (end 180.263971 128.087513) (width 0.4) (layer B.Cu) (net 2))
 (segment (start 178.69 127.635) (end 179.811458 127.635) (width 0.4) (layer B.Cu) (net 2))
 (segment (start 182.7276 134.62) (end 182.88 134.62) (width 0.4) (layer B.Cu) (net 2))
 (segment (start 180.863981 130.216381) (end 180.86398 127.83898) (width 0.4) (layer B.Cu) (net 3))
 (segment (start 182.7276 132.08) (end 180.863981 130.216381) (width 0.4) (layer B.Cu) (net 3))
 (segment (start 180.86398 127.83898) (end 179.39 126.365) (width 0.4) (layer B.Cu) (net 3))
 (segment (start 182.88 132.08) (end 182.7276 132.08) (width 0.4) (layer B.Cu) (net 3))
 (segment (start 179.39 126.365) (end 178.69 126.365) (width 0.4) (layer B.Cu) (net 3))
 (segment (start 178.69 126.365) (end 179.39 126.365) (width 0.4) (layer F.Cu) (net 3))
 (segment (start 179.39 126.365) (end 180.86398 127.83898) (width 0.4) (layer F.Cu) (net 3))
 (segment (start 180.86398 127.83898) (end 180.86398 130.21638) (width 0.4) (layer F.Cu) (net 3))
 (segment (start 180.86398 130.21638) (end 182.7276 132.08) (width 0.4) (layer F.Cu) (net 3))
 (segment (start 182.7276 132.08) (end 182.88 132.08) (width 0.4) (layer F.Cu) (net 3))
 (segment (start 181.46399 127.127) (end 181.46399 128.27639) (width 0.4) (layer B.Cu) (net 4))
 (segment (start 181.46399 127.127) (end 181.422 127.127) (width 0.4) (layer B.Cu) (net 4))
 (segment (start 179.39 125.095) (end 178.69 125.095) (width 0.4) (layer B.Cu) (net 4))
 (segment (start 181.422 127.127) (end 179.39 125.095) (width 0.4) (layer B.Cu) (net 4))
 (segment (start 181.46399 128.27639) (end 182.7276 129.54) (width 0.4) (layer B.Cu) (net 4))
 (segment (start 182.7276 129.54) (end 182.88 129.54) (width 0.4) (layer B.Cu) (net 4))
 (segment (start 178.69 125.095) (end 179.39 125.095) (width 0.4) (layer F.Cu) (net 4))
 (segment (start 179.39 125.095) (end 181.46399 127.16899) (width 0.4) (layer F.Cu) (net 4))
 (segment (start 181.46399 127.16899) (end 181.46399 128.27639) (width 0.4) (layer F.Cu) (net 4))
 (segment (start 181.46399 128.27639) (end 182.7276 129.54) (width 0.4) (layer F.Cu) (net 4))
 (segment (start 182.7276 129.54) (end 182.88 129.54) (width 0.4) (layer F.Cu) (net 4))
 (segment (start 182.88 127) (end 182.565 127) (width 0.4) (layer F.Cu) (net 5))
 (segment (start 179.39 123.825) (end 178.69 123.825) (width 0.4) (layer F.Cu) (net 5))
 (segment (start 182.565 127) (end 179.39 123.825) (width 0.4) (layer F.Cu) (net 5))
 (segment (start 179.7558 123.825) (end 179.7558 124.0282) (width 0.4) (layer B.Cu) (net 5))
 (segment (start 179.7558 124.0282) (end 182.7276 127) (width 0.4) (layer B.Cu) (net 5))
 (segment (start 182.7276 127) (end 182.88 127) (width 0.4) (layer B.Cu) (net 5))
 (segment (start 178.69 123.825) (end 179.7558 123.825) (width 0.4) (layer B.Cu) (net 5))
 (segment (start 178.69 121.285) (end 182.245 121.285) (width 0.4) (layer F.Cu) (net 7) (status 30))
 (segment (start 182.245 121.285) (end 182.88 121.92) (width 0.4) (layer F.Cu) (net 7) (status 30))
 (segment (start 178.69 120.015) (end 182.245 120.015) (width 0.4) (layer F.Cu) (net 8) (status 30))
 (segment (start 182.245 120.015) (end 182.88 119.38) (width 0.4) (layer F.Cu) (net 8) (status 30))
 (segment (start 178.69 118.745) (end 180.975 118.745) (width 0.4) (layer F.Cu) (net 9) (status 10))
 (segment (start 180.975 118.745) (end 182.88 116.84) (width 0.4) (layer F.Cu) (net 9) (status 20))
 (segment (start 165.1 114.3) (end 165.1 114.554) (width 0.4) (layer F.Cu) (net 2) (status 30))
 (segment (start 165.1 114.554) (end 168.021 117.475) (width 0.4) (layer F.Cu) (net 2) (status 10))
 (segment (start 168.021 117.475) (end 169.29 117.475) (width 0.4) (layer F.Cu) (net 2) (status 20))
 (segment (start 169.29 118.745) (end 167.005 118.745) (width 0.4) (layer F.Cu) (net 17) (status 10))
 (segment (start 167.005 118.745) (end 165.1 116.84) (width 0.4) (layer F.Cu) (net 17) (status 20))
 (segment (start 169.29 120.015) (end 165.735 120.015) (width 0.4) (layer F.Cu) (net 18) (status 30))
 (segment (start 165.735 120.015) (end 165.1 119.38) (width 0.4) (layer F.Cu) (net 18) (status 30))
 (segment (start 169.29 121.285) (end 165.735 121.285) (width 0.4) (layer F.Cu) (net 19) (status 30))
 (segment (start 165.735 121.285) (end 165.1 121.92) (width 0.4) (layer F.Cu) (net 19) (status 30))
 (segment (start 169.29 122.555) (end 167.005 122.555) (width 0.4) (layer F.Cu) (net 20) (status 10))
 (segment (start 167.005 122.555) (end 165.1 124.46) (width 0.4) (layer F.Cu) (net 20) (status 20))
 (segment (start 169.29 123.825) (end 168.275 123.825) (width 0.4) (layer F.Cu) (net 21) (status 10))
 (segment (start 168.275 123.825) (end 165.1 127) (width 0.4) (layer F.Cu) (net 21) (status 20))
 (segment (start 167.8686 125.124006) (end 167.8686 125.1164) (width 0.4) (layer B.Cu) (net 22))
 (segment (start 167.8686 125.1164) (end 167.89 125.095) (width 0.4) (layer B.Cu) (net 22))
 (segment (start 167.89 125.095) (end 169.29 125.095) (width 0.4) (layer B.Cu) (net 22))
 (segment (start 166.51601 126.476596) (end 167.8686 125.124006) (width 0.4) (layer B.Cu) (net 22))
 (segment (start 165.1 129.54) (end 165.2524 129.54) (width 0.4) (layer B.Cu) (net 22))
 (segment (start 165.2524 129.54) (end 166.51601 128.27639) (width 0.4) (layer B.Cu) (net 22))
 (segment (start 166.51601 128.27639) (end 166.51601 126.476596) (width 0.4) (layer B.Cu) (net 22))
 (segment (start 166.527571 126.420971) (end 166.527571 128.264829) (width 0.4) (layer F.Cu) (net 22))
 (segment (start 166.527571 128.264829) (end 165.2524 129.54) (width 0.4) (layer F.Cu) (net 22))
 (segment (start 165.2524 129.54) (end 165.1 129.54) (width 0.4) (layer F.Cu) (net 22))
 (segment (start 167.345542 125.603) (end 166.527571 126.420971) (width 0.4) (layer F.Cu) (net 22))
 (segment (start 169.29 125.095) (end 167.89 125.095) (width 0.4) (layer F.Cu) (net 22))
 (segment (start 167.89 125.095) (end 167.382 125.603) (width 0.4) (layer F.Cu) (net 22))
 (segment (start 167.382 125.603) (end 167.345542 125.603) (width 0.4) (layer F.Cu) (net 22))
 (segment (start 169.29 126.365) (end 167.89 126.365) (width 0.4) (layer B.Cu) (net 23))
 (segment (start 165.2524 132.08) (end 165.1 132.08) (width 0.4) (layer B.Cu) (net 23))
 (segment (start 167.89 126.365) (end 167.11602 127.13898) (width 0.4) (layer B.Cu) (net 23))
 (segment (start 167.11602 130.21638) (end 165.2524 132.08) (width 0.4) (layer B.Cu) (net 23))
 (segment (start 167.11602 127.13898) (end 167.11602 130.21638) (width 0.4) (layer B.Cu) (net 23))
 (segment (start 169.29 126.365) (end 167.89 126.365) (width 0.4) (layer F.Cu) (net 23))
 (segment (start 167.89 126.365) (end 167.127581 127.127419) (width 0.4) (layer F.Cu) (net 23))
 (segment (start 167.127581 130.204819) (end 165.2524 132.08) (width 0.4) (layer F.Cu) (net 23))
 (segment (start 165.2524 132.08) (end 165.1 132.08) (width 0.4) (layer F.Cu) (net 23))
 (segment (start 167.127581 127.127419) (end 167.127581 130.204819) (width 0.4) (layer F.Cu) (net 23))
 (segment (start 165.1 134.62) (end 165.2524 134.62) (width 0.4) (layer B.Cu) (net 24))
 (segment (start 167.71603 128.50897) (end 168.59 127.635) (width 0.4) (layer B.Cu) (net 24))
 (segment (start 165.2524 134.62) (end 167.71603 132.15637) (width 0.4) (layer B.Cu) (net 24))
 (segment (start 167.71603 132.15637) (end 167.71603 128.50897) (width 0.4) (layer B.Cu) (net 24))
 (segment (start 168.59 127.635) (end 169.29 127.635) (width 0.4) (layer B.Cu) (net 24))
 (segment (start 169.29 127.635) (end 168.59 127.635) (width 0.4) (layer F.Cu) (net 24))
 (segment (start 165.2524 134.62) (end 165.1 134.62) (width 0.4) (layer F.Cu) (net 24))
 (segment (start 168.59 127.635) (end 167.727591 128.497409) (width 0.4) (layer F.Cu) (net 24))
 (segment (start 167.727591 128.497409) (end 167.727591 132.144809) (width 0.4) (layer F.Cu) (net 24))
 (segment (start 167.727591 132.144809) (end 165.2524 134.62) (width 0.4) (layer F.Cu) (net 24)))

